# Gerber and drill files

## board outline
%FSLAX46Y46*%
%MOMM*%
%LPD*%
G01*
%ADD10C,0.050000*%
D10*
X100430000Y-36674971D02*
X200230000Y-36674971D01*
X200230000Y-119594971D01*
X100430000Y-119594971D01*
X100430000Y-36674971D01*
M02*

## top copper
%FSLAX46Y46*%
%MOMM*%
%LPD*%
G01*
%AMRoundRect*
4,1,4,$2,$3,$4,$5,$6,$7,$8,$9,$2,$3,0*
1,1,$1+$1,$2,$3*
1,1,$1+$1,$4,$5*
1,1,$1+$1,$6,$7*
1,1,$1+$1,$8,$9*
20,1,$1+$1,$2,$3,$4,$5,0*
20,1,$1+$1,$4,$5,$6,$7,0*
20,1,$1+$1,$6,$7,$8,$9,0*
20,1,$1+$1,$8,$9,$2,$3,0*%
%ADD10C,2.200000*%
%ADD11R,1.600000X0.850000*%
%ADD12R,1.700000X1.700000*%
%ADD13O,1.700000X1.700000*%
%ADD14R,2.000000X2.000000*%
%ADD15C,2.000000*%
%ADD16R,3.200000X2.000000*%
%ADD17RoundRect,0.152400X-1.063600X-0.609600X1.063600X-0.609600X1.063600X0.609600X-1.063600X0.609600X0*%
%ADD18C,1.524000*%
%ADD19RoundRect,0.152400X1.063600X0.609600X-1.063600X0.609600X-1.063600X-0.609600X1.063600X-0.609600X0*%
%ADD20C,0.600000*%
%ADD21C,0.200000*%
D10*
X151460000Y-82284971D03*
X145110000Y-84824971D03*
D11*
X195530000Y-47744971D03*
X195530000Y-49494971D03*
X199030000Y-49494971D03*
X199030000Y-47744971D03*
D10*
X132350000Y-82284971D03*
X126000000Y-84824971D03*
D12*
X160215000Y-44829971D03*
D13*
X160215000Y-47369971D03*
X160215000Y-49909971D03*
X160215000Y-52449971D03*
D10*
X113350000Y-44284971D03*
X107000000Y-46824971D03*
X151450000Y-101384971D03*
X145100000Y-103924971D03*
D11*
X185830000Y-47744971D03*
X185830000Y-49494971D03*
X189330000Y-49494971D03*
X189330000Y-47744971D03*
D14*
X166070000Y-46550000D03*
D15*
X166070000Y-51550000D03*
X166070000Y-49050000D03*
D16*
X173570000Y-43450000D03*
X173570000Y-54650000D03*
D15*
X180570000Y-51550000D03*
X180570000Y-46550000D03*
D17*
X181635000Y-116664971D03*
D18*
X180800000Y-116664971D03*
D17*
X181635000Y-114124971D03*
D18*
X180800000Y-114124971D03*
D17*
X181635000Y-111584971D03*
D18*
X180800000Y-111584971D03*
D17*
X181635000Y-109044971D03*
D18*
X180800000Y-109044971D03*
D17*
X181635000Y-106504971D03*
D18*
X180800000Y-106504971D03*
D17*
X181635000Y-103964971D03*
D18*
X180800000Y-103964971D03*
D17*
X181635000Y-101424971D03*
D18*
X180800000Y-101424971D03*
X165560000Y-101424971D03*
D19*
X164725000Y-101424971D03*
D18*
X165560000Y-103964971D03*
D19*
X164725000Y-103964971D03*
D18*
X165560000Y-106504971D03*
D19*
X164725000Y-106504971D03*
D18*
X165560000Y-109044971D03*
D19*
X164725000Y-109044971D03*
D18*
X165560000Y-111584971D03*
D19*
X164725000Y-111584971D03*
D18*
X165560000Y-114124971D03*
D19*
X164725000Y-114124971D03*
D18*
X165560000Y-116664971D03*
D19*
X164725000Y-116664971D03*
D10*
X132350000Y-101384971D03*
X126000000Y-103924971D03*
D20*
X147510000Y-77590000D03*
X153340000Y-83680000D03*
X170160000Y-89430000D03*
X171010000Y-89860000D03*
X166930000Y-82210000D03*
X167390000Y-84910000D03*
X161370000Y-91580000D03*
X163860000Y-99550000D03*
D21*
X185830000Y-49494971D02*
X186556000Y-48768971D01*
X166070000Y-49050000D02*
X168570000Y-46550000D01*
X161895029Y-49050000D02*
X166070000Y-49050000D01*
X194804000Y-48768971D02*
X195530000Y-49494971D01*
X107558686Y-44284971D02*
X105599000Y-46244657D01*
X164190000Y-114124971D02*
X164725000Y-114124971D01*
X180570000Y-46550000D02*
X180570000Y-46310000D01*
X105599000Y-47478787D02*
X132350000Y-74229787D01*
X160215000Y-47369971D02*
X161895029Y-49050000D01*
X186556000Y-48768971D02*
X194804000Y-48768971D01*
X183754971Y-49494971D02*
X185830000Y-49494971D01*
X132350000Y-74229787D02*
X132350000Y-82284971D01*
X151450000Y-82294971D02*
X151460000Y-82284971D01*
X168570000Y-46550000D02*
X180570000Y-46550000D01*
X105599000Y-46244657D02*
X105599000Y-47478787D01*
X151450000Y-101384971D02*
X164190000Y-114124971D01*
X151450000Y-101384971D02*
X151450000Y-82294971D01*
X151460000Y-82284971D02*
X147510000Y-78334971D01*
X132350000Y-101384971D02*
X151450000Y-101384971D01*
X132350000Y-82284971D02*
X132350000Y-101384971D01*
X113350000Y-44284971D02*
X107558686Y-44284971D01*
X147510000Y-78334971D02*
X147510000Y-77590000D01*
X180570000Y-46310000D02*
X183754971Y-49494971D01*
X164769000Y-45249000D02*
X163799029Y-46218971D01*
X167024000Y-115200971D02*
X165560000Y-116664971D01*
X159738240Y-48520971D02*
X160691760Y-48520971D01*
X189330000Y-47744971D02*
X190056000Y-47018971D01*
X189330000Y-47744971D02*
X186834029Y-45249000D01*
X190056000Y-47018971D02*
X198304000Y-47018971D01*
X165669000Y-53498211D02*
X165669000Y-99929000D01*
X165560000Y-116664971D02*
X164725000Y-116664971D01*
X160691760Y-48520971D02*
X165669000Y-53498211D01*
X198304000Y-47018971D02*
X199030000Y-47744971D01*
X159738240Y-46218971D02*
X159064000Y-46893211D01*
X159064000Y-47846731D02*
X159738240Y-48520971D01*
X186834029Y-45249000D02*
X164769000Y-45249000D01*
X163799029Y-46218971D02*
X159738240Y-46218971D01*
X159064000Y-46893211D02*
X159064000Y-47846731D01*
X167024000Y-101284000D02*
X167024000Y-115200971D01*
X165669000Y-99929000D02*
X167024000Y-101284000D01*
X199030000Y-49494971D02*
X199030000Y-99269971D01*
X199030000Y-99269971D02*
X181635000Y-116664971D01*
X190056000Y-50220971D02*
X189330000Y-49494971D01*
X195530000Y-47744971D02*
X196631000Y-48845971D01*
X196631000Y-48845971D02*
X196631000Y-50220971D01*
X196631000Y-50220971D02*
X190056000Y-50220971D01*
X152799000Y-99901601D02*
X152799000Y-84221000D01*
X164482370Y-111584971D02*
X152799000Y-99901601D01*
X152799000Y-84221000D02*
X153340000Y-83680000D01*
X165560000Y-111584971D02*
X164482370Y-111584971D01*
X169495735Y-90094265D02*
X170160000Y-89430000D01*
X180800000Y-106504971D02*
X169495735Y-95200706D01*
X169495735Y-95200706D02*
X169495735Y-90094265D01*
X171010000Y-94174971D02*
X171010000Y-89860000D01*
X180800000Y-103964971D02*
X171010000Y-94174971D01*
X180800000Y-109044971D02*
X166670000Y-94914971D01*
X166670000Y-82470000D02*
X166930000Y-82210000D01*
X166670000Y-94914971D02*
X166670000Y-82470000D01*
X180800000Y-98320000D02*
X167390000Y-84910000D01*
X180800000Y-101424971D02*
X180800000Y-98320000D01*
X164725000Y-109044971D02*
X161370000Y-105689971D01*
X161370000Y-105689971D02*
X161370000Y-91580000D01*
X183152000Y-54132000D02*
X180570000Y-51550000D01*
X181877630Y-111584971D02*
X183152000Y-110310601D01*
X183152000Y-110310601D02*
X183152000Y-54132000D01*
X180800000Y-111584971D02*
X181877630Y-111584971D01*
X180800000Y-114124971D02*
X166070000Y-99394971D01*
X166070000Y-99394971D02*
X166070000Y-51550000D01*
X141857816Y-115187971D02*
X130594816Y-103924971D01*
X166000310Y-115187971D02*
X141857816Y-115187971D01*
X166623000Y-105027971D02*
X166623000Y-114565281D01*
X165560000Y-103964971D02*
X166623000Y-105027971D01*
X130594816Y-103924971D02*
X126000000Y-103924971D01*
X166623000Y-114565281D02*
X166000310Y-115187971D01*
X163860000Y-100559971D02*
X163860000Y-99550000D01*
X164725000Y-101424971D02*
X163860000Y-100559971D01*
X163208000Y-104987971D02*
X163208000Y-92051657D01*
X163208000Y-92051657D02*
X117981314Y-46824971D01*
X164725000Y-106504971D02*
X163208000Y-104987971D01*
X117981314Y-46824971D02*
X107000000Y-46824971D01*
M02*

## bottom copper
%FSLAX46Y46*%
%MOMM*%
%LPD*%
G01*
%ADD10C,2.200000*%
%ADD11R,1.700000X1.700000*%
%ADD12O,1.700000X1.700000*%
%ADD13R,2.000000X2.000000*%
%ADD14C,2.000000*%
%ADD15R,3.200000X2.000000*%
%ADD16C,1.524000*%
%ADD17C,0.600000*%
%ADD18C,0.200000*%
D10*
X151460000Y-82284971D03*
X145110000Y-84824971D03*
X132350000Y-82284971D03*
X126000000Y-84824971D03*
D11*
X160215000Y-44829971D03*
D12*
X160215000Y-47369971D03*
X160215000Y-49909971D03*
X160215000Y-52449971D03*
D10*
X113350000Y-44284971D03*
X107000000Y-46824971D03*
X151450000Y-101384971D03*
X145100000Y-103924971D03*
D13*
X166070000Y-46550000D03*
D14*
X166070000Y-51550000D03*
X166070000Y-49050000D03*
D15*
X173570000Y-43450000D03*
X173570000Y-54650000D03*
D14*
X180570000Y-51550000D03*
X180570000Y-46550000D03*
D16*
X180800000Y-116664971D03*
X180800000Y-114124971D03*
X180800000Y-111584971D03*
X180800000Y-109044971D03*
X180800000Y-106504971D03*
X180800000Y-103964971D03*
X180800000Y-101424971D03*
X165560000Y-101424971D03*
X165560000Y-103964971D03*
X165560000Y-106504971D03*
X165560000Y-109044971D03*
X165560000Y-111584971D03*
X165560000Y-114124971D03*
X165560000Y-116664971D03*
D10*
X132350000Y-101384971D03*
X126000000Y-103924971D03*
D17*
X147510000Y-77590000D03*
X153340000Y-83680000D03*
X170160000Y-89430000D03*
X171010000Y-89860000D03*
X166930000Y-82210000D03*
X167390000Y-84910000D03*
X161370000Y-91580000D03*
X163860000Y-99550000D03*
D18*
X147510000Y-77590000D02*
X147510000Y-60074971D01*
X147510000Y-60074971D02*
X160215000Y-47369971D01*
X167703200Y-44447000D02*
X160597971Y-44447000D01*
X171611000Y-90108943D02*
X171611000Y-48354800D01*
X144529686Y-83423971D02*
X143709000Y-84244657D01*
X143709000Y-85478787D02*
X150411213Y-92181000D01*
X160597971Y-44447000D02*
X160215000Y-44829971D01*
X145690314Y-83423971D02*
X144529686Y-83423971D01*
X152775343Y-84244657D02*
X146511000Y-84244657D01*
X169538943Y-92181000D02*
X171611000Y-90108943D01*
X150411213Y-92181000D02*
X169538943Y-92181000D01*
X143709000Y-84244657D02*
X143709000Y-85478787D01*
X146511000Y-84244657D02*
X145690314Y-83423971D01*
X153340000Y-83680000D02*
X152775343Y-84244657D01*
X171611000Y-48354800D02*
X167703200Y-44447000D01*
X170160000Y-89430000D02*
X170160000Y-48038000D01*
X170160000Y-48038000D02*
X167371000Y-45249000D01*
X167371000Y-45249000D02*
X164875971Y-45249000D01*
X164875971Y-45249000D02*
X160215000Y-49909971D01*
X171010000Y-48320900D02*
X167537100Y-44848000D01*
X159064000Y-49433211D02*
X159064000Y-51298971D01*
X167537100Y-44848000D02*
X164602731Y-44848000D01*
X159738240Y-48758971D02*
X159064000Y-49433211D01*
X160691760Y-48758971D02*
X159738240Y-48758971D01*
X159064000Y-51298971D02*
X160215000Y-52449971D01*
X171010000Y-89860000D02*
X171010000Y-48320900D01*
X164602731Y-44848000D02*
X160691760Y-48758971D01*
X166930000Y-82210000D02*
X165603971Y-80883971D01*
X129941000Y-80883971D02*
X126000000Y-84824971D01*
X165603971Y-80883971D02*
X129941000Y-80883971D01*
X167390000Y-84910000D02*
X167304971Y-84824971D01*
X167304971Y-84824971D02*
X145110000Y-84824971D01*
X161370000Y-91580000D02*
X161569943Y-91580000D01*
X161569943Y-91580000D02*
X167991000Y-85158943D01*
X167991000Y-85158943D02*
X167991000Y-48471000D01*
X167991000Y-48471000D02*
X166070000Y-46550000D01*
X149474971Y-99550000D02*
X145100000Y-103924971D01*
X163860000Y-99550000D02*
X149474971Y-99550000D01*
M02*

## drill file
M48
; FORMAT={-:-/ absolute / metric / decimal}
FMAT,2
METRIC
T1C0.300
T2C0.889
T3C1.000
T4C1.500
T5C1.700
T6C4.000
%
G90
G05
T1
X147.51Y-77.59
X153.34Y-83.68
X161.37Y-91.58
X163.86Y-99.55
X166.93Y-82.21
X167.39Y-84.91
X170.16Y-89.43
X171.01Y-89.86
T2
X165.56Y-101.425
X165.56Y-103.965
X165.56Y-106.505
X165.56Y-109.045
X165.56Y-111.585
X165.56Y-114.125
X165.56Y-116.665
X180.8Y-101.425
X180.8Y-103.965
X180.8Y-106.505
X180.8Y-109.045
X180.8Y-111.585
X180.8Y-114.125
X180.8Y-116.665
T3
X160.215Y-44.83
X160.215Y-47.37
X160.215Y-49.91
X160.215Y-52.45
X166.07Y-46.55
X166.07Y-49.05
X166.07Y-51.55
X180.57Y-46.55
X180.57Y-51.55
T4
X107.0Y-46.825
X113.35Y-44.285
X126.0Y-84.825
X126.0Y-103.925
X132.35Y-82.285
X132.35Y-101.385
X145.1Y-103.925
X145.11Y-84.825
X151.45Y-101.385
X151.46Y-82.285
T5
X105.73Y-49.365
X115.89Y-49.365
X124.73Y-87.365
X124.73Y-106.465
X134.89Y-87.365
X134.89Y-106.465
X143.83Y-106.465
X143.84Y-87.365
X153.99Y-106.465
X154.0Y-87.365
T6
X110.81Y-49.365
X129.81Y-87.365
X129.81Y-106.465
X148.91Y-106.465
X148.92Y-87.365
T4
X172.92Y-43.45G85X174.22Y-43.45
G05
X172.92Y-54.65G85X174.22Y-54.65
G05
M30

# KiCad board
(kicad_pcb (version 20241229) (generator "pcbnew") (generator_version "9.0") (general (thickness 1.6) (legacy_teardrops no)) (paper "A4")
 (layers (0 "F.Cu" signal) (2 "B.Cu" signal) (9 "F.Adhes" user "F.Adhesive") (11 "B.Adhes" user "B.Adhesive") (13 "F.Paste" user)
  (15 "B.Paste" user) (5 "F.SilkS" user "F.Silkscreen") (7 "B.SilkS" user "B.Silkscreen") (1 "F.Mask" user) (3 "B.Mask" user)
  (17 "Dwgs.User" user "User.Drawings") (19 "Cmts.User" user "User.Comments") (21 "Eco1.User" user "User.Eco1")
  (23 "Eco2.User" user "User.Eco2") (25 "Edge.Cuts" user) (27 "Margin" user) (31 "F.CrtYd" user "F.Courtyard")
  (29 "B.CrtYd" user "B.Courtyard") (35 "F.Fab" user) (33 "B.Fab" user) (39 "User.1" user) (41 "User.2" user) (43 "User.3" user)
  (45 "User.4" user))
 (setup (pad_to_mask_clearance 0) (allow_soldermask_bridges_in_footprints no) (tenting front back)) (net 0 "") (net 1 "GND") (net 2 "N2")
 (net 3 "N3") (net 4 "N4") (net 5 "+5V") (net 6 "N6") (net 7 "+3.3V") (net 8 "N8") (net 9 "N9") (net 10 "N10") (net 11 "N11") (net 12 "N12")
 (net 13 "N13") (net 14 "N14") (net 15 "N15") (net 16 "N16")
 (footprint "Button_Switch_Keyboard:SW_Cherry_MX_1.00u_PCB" (layer "F.Cu") (at 151.46 82.284971)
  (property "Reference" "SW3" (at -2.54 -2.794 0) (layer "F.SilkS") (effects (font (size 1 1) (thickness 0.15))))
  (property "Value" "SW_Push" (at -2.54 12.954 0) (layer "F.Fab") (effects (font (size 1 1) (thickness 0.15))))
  (pad "" np_thru_hole circle (at -7.62 5.08) (size 1.7 1.7) (drill 1.7) (layers "*.Cu" "*.Mask"))
  (pad "" np_thru_hole circle (at -2.54 5.08) (size 4 4) (drill 4) (layers "*.Cu" "*.Mask"))
  (pad "" np_thru_hole circle (at 2.54 5.08) (size 1.7 1.7) (drill 1.7) (layers "*.Cu" "*.Mask"))
  (pad "1" thru_hole circle (at 0 0) (size 2.2 2.2) (drill 1.5) (layers "*.Cu" "*.Mask") (remove_unused_layers no) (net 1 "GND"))
  (pad "2" thru_hole circle (at -6.35 2.54) (size 2.2 2.2) (drill 1.5) (layers "*.Cu" "*.Mask") (remove_unused_layers no) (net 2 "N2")))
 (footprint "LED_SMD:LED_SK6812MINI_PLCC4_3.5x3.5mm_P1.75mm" (layer "F.Cu") (at 197.28 48.619971)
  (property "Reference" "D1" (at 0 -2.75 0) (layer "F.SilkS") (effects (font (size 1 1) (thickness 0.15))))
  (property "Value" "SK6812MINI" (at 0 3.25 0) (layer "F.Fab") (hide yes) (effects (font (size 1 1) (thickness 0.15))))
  (pad "1" smd rect (at -1.75 -0.875) (size 1.6 0.85) (layers "F.Cu" "F.Mask" "F.Paste") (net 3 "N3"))
  (pad "2" smd rect (at -1.75 0.875) (size 1.6 0.85) (layers "F.Cu" "F.Mask" "F.Paste") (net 1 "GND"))
  (pad "3" smd rect (at 1.75 0.875) (size 1.6 0.85) (layers "F.Cu" "F.Mask" "F.Paste") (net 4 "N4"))
  (pad "4" smd rect (at 1.75 -0.875) (size 1.6 0.85) (layers "F.Cu" "F.Mask" "F.Paste") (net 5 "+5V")))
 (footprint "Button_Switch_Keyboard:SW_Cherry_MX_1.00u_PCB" (layer "F.Cu") (at 132.35 82.284971)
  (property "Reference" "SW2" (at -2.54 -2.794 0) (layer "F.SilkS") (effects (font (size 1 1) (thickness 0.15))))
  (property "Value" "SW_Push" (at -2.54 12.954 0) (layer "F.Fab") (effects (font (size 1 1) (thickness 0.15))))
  (pad "" np_thru_hole circle (at -7.62 5.08) (size 1.7 1.7) (drill 1.7) (layers "*.Cu" "*.Mask"))
  (pad "" np_thru_hole circle (at -2.54 5.08) (size 4 4) (drill 4) (layers "*.Cu" "*.Mask"))
  (pad "" np_thru_hole circle (at 2.54 5.08) (size 1.7 1.7) (drill 1.7) (layers "*.Cu" "*.Mask"))
  (pad "1" thru_hole circle (at 0 0) (size 2.2 2.2) (drill 1.5) (layers "*.Cu" "*.Mask") (remove_unused_layers no) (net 1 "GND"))
  (pad "2" thru_hole circle (at -6.35 2.54) (size 2.2 2.2) (drill 1.5) (layers "*.Cu" "*.Mask") (remove_unused_layers no) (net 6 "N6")))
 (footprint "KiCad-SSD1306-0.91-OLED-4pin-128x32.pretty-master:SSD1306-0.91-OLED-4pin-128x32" (layer "F.Cu") (at 123.715 42.639971)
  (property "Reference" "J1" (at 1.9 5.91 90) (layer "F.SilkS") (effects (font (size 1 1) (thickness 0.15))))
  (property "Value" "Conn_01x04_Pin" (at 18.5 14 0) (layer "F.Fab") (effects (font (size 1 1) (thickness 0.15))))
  (pad "1" thru_hole rect (at 36.5 2.19) (size 1.7 1.7) (drill 1) (layers "*.Cu" "*.Mask") (remove_unused_layers no) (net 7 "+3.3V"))
  (pad "2" thru_hole oval (at 36.5 4.73) (size 1.7 1.7) (drill 1) (layers "*.Cu" "*.Mask") (remove_unused_layers no) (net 1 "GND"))
  (pad "3" thru_hole oval (at 36.5 7.27) (size 1.7 1.7) (drill 1) (layers "*.Cu" "*.Mask") (remove_unused_layers no) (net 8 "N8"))
  (pad "4" thru_hole oval (at 36.5 9.81) (size 1.7 1.7) (drill 1) (layers "*.Cu" "*.Mask") (remove_unused_layers no) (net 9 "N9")))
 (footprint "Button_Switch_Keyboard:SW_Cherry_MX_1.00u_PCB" (layer "F.Cu") (at 113.35 44.284971)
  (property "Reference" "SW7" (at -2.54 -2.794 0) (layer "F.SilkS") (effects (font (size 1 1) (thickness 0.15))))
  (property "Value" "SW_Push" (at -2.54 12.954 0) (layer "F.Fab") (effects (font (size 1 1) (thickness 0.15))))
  (pad "" np_thru_hole circle (at -7.62 5.08) (size 1.7 1.7) (drill 1.7) (layers "*.Cu" "*.Mask"))
  (pad "" np_thru_hole circle (at -2.54 5.08) (size 4 4) (drill 4) (layers "*.Cu" "*.Mask"))
  (pad "" np_thru_hole circle (at 2.54 5.08) (size 1.7 1.7) (drill 1.7) (layers "*.Cu" "*.Mask"))
  (pad "1" thru_hole circle (at 0 0) (size 2.2 2.2) (drill 1.5) (layers "*.Cu" "*.Mask") (remove_unused_layers no) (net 1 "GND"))
  (pad "2" thru_hole circle (at -6.35 2.54) (size 2.2 2.2) (drill 1.5) (layers "*.Cu" "*.Mask") (remove_unused_layers no) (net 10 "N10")))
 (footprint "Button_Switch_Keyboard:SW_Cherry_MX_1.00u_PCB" (layer "F.Cu") (at 151.45 101.384971)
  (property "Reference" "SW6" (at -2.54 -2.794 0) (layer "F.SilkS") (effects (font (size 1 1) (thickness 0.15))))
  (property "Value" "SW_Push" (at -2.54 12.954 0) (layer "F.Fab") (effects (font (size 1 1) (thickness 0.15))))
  (pad "" np_thru_hole circle (at -7.62 5.08) (size 1.7 1.7) (drill 1.7) (layers "*.Cu" "*.Mask"))
  (pad "" np_thru_hole circle (at -2.54 5.08) (size 4 4) (drill 4) (layers "*.Cu" "*.Mask"))
  (pad "" np_thru_hole circle (at 2.54 5.08) (size 1.7 1.7) (drill 1.7) (layers "*.Cu" "*.Mask"))
  (pad "1" thru_hole circle (at 0 0) (size 2.2 2.2) (drill 1.5) (layers "*.Cu" "*.Mask") (remove_unused_layers no) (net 1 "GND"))
  (pad "2" thru_hole circle (at -6.35 2.54) (size 2.2 2.2) (drill 1.5) (layers "*.Cu" "*.Mask") (remove_unused_layers no) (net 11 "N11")))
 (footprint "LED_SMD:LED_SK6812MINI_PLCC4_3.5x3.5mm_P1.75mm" (layer "F.Cu") (at 187.58 48.619971)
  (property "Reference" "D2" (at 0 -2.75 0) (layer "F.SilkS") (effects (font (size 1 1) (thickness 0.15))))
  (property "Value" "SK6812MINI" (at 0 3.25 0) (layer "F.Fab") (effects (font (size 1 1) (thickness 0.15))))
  (pad "1" smd rect (at -1.75 -0.875) (size 1.6 0.85) (layers "F.Cu" "F.Mask" "F.Paste") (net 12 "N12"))
  (pad "2" smd rect (at -1.75 0.875) (size 1.6 0.85) (layers "F.Cu" "F.Mask" "F.Paste") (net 1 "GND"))
  (pad "3" smd rect (at 1.75 0.875) (size 1.6 0.85) (layers "F.Cu" "F.Mask" "F.Paste") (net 3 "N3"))
  (pad "4" smd rect (at 1.75 -0.875) (size 1.6 0.85) (layers "F.Cu" "F.Mask" "F.Paste") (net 5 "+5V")))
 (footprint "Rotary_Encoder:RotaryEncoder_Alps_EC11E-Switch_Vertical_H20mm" (layer "F.Cu") (at 166.07 46.55)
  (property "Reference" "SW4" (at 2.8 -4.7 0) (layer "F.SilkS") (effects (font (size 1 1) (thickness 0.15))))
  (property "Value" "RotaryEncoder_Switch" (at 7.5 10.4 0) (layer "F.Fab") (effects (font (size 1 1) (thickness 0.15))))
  (pad "A" thru_hole rect (at 0 0) (size 2 2) (drill 1) (layers "*.Cu" "*.Mask") (remove_unused_layers no) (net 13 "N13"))
  (pad "B" thru_hole circle (at 0 5) (size 2 2) (drill 1) (layers "*.Cu" "*.Mask") (remove_unused_layers no) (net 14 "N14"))
  (pad "C" thru_hole circle (at 0 2.5) (size 2 2) (drill 1) (layers "*.Cu" "*.Mask") (remove_unused_layers no) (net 1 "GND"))
  (pad "MP" thru_hole rect (at 7.5 -3.1) (size 3.2 2) (drill oval 2.8 1.5) (layers "*.Cu" "*.Mask") (remove_unused_layers no))
  (pad "MP" thru_hole rect (at 7.5 8.1) (size 3.2 2) (drill oval 2.8 1.5) (layers "*.Cu" "*.Mask") (remove_unused_layers no))
  (pad "S1" thru_hole circle (at 14.5 5) (size 2 2) (drill 1) (layers "*.Cu" "*.Mask") (remove_unused_layers no) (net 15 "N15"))
  (pad "S2" thru_hole circle (at 14.5 0) (size 2 2) (drill 1) (layers "*.Cu" "*.Mask") (remove_unused_layers no) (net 1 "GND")))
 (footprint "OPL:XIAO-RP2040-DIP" (layer "F.Cu") (at 173.18 109.044971 180)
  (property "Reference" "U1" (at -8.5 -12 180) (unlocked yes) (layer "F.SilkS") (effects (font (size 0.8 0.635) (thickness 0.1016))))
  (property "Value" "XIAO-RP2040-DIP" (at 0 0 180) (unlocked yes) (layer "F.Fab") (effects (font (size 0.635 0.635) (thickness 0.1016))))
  (pad "1" smd roundrect (at -8.455 -7.62) (size 2.432 1.524) (layers "F.Cu" "F.Mask") (roundrect_rratio 0.1) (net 4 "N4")
   (thermal_bridge_angle 45))
  (pad "1" thru_hole circle (at -7.62 -7.62) (size 1.524 1.524) (drill 0.889) (layers "*.Cu" "*.Mask") (remove_unused_layers no)
   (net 4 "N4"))
  (pad "2" smd roundrect (at -8.455 -5.08) (size 2.432 1.524) (layers "F.Cu" "F.Mask") (roundrect_rratio 0.1) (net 14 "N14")
   (thermal_bridge_angle 45))
  (pad "2" thru_hole circle (at -7.62 -5.08) (size 1.524 1.524) (drill 0.889) (layers "*.Cu" "*.Mask") (remove_unused_layers no)
   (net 14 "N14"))
  (pad "3" smd roundrect (at -8.455 -2.54) (size 2.432 1.524) (layers "F.Cu" "F.Mask") (roundrect_rratio 0.1) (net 15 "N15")
   (thermal_bridge_angle 45))
  (pad "3" thru_hole circle (at -7.62 -2.54) (size 1.524 1.524) (drill 0.889) (layers "*.Cu" "*.Mask") (remove_unused_layers no)
   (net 15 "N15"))
  (pad "4" smd roundrect (at -8.455 0) (size 2.432 1.524) (layers "F.Cu" "F.Mask") (roundrect_rratio 0.1) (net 6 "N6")
   (thermal_bridge_angle 45))
  (pad "4" thru_hole circle (at -7.62 0) (size 1.524 1.524) (drill 0.889) (layers "*.Cu" "*.Mask") (remove_unused_layers no) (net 6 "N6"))
  (pad "5" smd roundrect (at -8.455 2.54) (size 2.432 1.524) (layers "F.Cu" "F.Mask") (roundrect_rratio 0.1) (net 8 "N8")
   (thermal_bridge_angle 45))
  (pad "5" thru_hole circle (at -7.62 2.54) (size 1.524 1.524) (drill 0.889) (layers "*.Cu" "*.Mask") (remove_unused_layers no) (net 8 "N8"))
  (pad "6" smd roundrect (at -8.455 5.08) (size 2.432 1.524) (layers "F.Cu" "F.Mask") (roundrect_rratio 0.1) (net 9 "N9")
   (thermal_bridge_angle 45))
  (pad "6" thru_hole circle (at -7.62 5.08) (size 1.524 1.524) (drill 0.889) (layers "*.Cu" "*.Mask") (remove_unused_layers no) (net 9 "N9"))
  (pad "7" smd roundrect (at -8.455 7.62) (size 2.432 1.524) (layers "F.Cu" "F.Mask") (roundrect_rratio 0.1) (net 2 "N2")
   (thermal_bridge_angle 45))
  (pad "7" thru_hole circle (at -7.62 7.62) (size 1.524 1.524) (drill 0.889) (layers "*.Cu" "*.Mask") (remove_unused_layers no) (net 2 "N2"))
  (pad "8" thru_hole circle (at 7.62 7.62 180) (size 1.524 1.524) (drill 0.889) (layers "*.Cu" "*.Mask") (remove_unused_layers no)
   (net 11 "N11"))
  (pad "8" smd roundrect (at 8.455 7.62 180) (size 2.432 1.524) (layers "F.Cu" "F.Mask") (roundrect_rratio 0.1) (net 11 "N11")
   (thermal_bridge_angle 45))
  (pad "9" thru_hole circle (at 7.62 5.08 180) (size 1.524 1.524) (drill 0.889) (layers "*.Cu" "*.Mask") (remove_unused_layers no)
   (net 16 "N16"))
  (pad "9" smd roundrect (at 8.455 5.08 180) (size 2.432 1.524) (layers "F.Cu" "F.Mask") (roundrect_rratio 0.1) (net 16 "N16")
   (thermal_bridge_angle 45))
  (pad "10" thru_hole circle (at 7.62 2.54 180) (size 1.524 1.524) (drill 0.889) (layers "*.Cu" "*.Mask") (remove_unused_layers no)
   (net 10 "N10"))
  (pad "10" smd roundrect (at 8.455 2.54 180) (size 2.432 1.524) (layers "F.Cu" "F.Mask") (roundrect_rratio 0.1) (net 10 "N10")
   (thermal_bridge_angle 45))
  (pad "11" thru_hole circle (at 7.62 0 180) (size 1.524 1.524) (drill 0.889) (layers "*.Cu" "*.Mask") (remove_unused_layers no)
   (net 13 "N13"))
  (pad "11" smd roundrect (at 8.455 0 180) (size 2.432 1.524) (layers "F.Cu" "F.Mask") (roundrect_rratio 0.1) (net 13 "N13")
   (thermal_bridge_angle 45))
  (pad "12" thru_hole circle (at 7.62 -2.54 180) (size 1.524 1.524) (drill 0.889) (layers "*.Cu" "*.Mask") (remove_unused_layers no)
   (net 7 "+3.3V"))
  (pad "12" smd roundrect (at 8.455 -2.54 180) (size 2.432 1.524) (layers "F.Cu" "F.Mask") (roundrect_rratio 0.1) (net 7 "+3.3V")
   (thermal_bridge_angle 45))
  (pad "13" thru_hole circle (at 7.62 -5.08 180) (size 1.524 1.524) (drill 0.889) (layers "*.Cu" "*.Mask") (remove_unused_layers no)
   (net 1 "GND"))
  (pad "13" smd roundrect (at 8.455 -5.08 180) (size 2.432 1.524) (layers "F.Cu" "F.Mask") (roundrect_rratio 0.1) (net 1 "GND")
   (thermal_bridge_angle 45))
  (pad "14" thru_hole circle (at 7.62 -7.62 180) (size 1.524 1.524) (drill 0.889) (layers "*.Cu" "*.Mask") (remove_unused_layers no)
   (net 5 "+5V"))
  (pad "14" smd roundrect (at 8.455 -7.62 180) (size 2.432 1.524) (layers "F.Cu" "F.Mask") (roundrect_rratio 0.1) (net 5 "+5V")
   (thermal_bridge_angle 45)))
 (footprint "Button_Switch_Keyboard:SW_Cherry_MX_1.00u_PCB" (layer "F.Cu") (at 132.35 101.384971)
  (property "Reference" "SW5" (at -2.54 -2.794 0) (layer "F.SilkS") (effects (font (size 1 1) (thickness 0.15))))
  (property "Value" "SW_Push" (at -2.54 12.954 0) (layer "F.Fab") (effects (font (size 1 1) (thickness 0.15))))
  (pad "" np_thru_hole circle (at -7.62 5.08) (size 1.7 1.7) (drill 1.7) (layers "*.Cu" "*.Mask"))
  (pad "" np_thru_hole circle (at -2.54 5.08) (size 4 4) (drill 4) (layers "*.Cu" "*.Mask"))
  (pad "" np_thru_hole circle (at 2.54 5.08) (size 1.7 1.7) (drill 1.7) (layers "*.Cu" "*.Mask"))
  (pad "1" thru_hole circle (at 0 0) (size 2.2 2.2) (drill 1.5) (layers "*.Cu" "*.Mask") (remove_unused_layers no) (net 1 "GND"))
  (pad "2" thru_hole circle (at -6.35 2.54) (size 2.2 2.2) (drill 1.5) (layers "*.Cu" "*.Mask") (remove_unused_layers no) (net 16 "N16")))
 (gr_rect (start 100.43 36.674971) (end 200.23 119.594971) (stroke (width 0.05) (type default)) (fill no) (layer "Edge.Cuts"))
 (segment (start 185.83 49.494971) (end 186.556 48.768971) (width 0.2) (layer "F.Cu") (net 1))
 (segment (start 166.07 49.05) (end 168.57 46.55) (width 0.2) (layer "F.Cu") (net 1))
 (segment (start 161.895029 49.05) (end 166.07 49.05) (width 0.2) (layer "F.Cu") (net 1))
 (segment (start 194.804 48.768971) (end 195.53 49.494971) (width 0.2) (layer "F.Cu") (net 1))
 (segment (start 107.558686 44.284971) (end 105.599 46.244657) (width 0.2) (layer "F.Cu") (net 1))
 (segment (start 164.19 114.124971) (end 164.725 114.124971) (width 0.2) (layer "F.Cu") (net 1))
 (segment (start 180.57 46.55) (end 180.57 46.31) (width 0.2) (layer "F.Cu") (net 1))
 (segment (start 105.599 47.478787) (end 132.35 74.229787) (width 0.2) (layer "F.Cu") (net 1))
 (segment (start 160.215 47.369971) (end 161.895029 49.05) (width 0.2) (layer "F.Cu") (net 1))
 (segment (start 186.556 48.768971) (end 194.804 48.768971) (width 0.2) (layer "F.Cu") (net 1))
 (segment (start 183.754971 49.494971) (end 185.83 49.494971) (width 0.2) (layer "F.Cu") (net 1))
 (segment (start 132.35 74.229787) (end 132.35 82.284971) (width 0.2) (layer "F.Cu") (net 1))
 (segment (start 151.45 82.294971) (end 151.46 82.284971) (width 0.2) (layer "F.Cu") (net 1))
 (segment (start 168.57 46.55) (end 180.57 46.55) (width 0.2) (layer "F.Cu") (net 1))
 (segment (start 105.599 46.244657) (end 105.599 47.478787) (width 0.2) (layer "F.Cu") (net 1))
 (segment (start 151.45 101.384971) (end 164.19 114.124971) (width 0.2) (layer "F.Cu") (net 1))
 (segment (start 151.45 101.384971) (end 151.45 82.294971) (width 0.2) (layer "F.Cu") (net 1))
 (segment (start 151.46 82.284971) (end 147.51 78.334971) (width 0.2) (layer "F.Cu") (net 1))
 (segment (start 132.35 101.384971) (end 151.45 101.384971) (width 0.2) (layer "F.Cu") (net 1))
 (segment (start 132.35 82.284971) (end 132.35 101.384971) (width 0.2) (layer "F.Cu") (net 1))
 (segment (start 113.35 44.284971) (end 107.558686 44.284971) (width 0.2) (layer "F.Cu") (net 1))
 (segment (start 147.51 78.334971) (end 147.51 77.59) (width 0.2) (layer "F.Cu") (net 1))
 (segment (start 180.57 46.31) (end 183.754971 49.494971) (width 0.2) (layer "F.Cu") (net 1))
 (via (at 147.51 77.59) (size 0.6) (drill 0.3) (layers "F.Cu" "B.Cu") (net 1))
 (segment (start 147.51 77.59) (end 147.51 60.074971) (width 0.2) (layer "B.Cu") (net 1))
 (segment (start 147.51 60.074971) (end 160.215 47.369971) (width 0.2) (layer "B.Cu") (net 1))
 (segment (start 164.769 45.249) (end 163.799029 46.218971) (width 0.2) (layer "F.Cu") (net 5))
 (segment (start 167.024 115.200971) (end 165.56 116.664971) (width 0.2) (layer "F.Cu") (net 5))
 (segment (start 159.73824 48.520971) (end 160.69176 48.520971) (width 0.2) (layer "F.Cu") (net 5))
 (segment (start 189.33 47.744971) (end 190.056 47.018971) (width 0.2) (layer "F.Cu") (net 5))
 (segment (start 189.33 47.744971) (end 186.834029 45.249) (width 0.2) (layer "F.Cu") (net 5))
 (segment (start 190.056 47.018971) (end 198.304 47.018971) (width 0.2) (layer "F.Cu") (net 5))
 (segment (start 165.669 53.498211) (end 165.669 99.929) (width 0.2) (layer "F.Cu") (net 5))
 (segment (start 165.56 116.664971) (end 164.725 116.664971) (width 0.2) (layer "F.Cu") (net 5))
 (segment (start 160.69176 48.520971) (end 165.669 53.498211) (width 0.2) (layer "F.Cu") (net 5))
 (segment (start 198.304 47.018971) (end 199.03 47.744971) (width 0.2) (layer "F.Cu") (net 5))
 (segment (start 159.73824 46.218971) (end 159.064 46.893211) (width 0.2) (layer "F.Cu") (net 5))
 (segment (start 159.064 47.846731) (end 159.73824 48.520971) (width 0.2) (layer "F.Cu") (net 5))
 (segment (start 186.834029 45.249) (end 164.769 45.249) (width 0.2) (layer "F.Cu") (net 5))
 (segment (start 163.799029 46.218971) (end 159.73824 46.218971) (width 0.2) (layer "F.Cu") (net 5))
 (segment (start 159.064 46.893211) (end 159.064 47.846731) (width 0.2) (layer "F.Cu") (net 5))
 (segment (start 167.024 101.284) (end 167.024 115.200971) (width 0.2) (layer "F.Cu") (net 5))
 (segment (start 165.669 99.929) (end 167.024 101.284) (width 0.2) (layer "F.Cu") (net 5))
 (segment (start 199.03 49.494971) (end 199.03 99.269971) (width 0.2) (layer "F.Cu") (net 4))
 (segment (start 199.03 99.269971) (end 181.635 116.664971) (width 0.2) (layer "F.Cu") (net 4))
 (segment (start 190.056 50.220971) (end 189.33 49.494971) (width 0.2) (layer "F.Cu") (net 3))
 (segment (start 195.53 47.744971) (end 196.631 48.845971) (width 0.2) (layer "F.Cu") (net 3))
 (segment (start 196.631 48.845971) (end 196.631 50.220971) (width 0.2) (layer "F.Cu") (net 3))
 (segment (start 196.631 50.220971) (end 190.056 50.220971) (width 0.2) (layer "F.Cu") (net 3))
 (segment (start 152.799 99.901601) (end 152.799 84.221) (width 0.2) (layer "F.Cu") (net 7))
 (segment (start 164.48237 111.584971) (end 152.799 99.901601) (width 0.2) (layer "F.Cu") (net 7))
 (segment (start 152.799 84.221) (end 153.34 83.68) (width 0.2) (layer "F.Cu") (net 7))
 (segment (start 165.56 111.584971) (end 164.48237 111.584971) (width 0.2) (layer "F.Cu") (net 7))
 (via (at 153.34 83.68) (size 0.6) (drill 0.3) (layers "F.Cu" "B.Cu") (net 7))
 (segment (start 167.7032 44.447) (end 160.597971 44.447) (width 0.2) (layer "B.Cu") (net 7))
 (segment (start 171.611 90.108943) (end 171.611 48.3548) (width 0.2) (layer "B.Cu") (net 7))
 (segment (start 144.529686 83.423971) (end 143.709 84.244657) (width 0.2) (layer "B.Cu") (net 7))
 (segment (start 143.709 85.478787) (end 150.411213 92.181) (width 0.2) (layer "B.Cu") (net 7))
 (segment (start 160.597971 44.447) (end 160.215 44.829971) (width 0.2) (layer "B.Cu") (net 7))
 (segment (start 145.690314 83.423971) (end 144.529686 83.423971) (width 0.2) (layer "B.Cu") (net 7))
 (segment (start 152.775343 84.244657) (end 146.511 84.244657) (width 0.2) (layer "B.Cu") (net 7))
 (segment (start 169.538943 92.181) (end 171.611 90.108943) (width 0.2) (layer "B.Cu") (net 7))
 (segment (start 150.411213 92.181) (end 169.538943 92.181) (width 0.2) (layer "B.Cu") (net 7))
 (segment (start 143.709 84.244657) (end 143.709 85.478787) (width 0.2) (layer "B.Cu") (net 7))
 (segment (start 146.511 84.244657) (end 145.690314 83.423971) (width 0.2) (layer "B.Cu") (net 7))
 (segment (start 153.34 83.68) (end 152.775343 84.244657) (width 0.2) (layer "B.Cu") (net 7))
 (segment (start 171.611 48.3548) (end 167.7032 44.447) (width 0.2) (layer "B.Cu") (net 7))
 (segment (start 169.495735 90.094265) (end 170.16 89.43) (width 0.2) (layer "F.Cu") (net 8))
 (segment (start 180.8 106.504971) (end 169.495735 95.200706) (width 0.2) (layer "F.Cu") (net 8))
 (segment (start 169.495735 95.200706) (end 169.495735 90.094265) (width 0.2) (layer "F.Cu") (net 8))
 (via (at 170.16 89.43) (size 0.6) (drill 0.3) (layers "F.Cu" "B.Cu") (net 8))
 (segment (start 170.16 89.43) (end 170.16 48.038) (width 0.2) (layer "B.Cu") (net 8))
 (segment (start 170.16 48.038) (end 167.371 45.249) (width 0.2) (layer "B.Cu") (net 8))
 (segment (start 167.371 45.249) (end 164.875971 45.249) (width 0.2) (layer "B.Cu") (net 8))
 (segment (start 164.875971 45.249) (end 160.215 49.909971) (width 0.2) (layer "B.Cu") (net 8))
 (segment (start 171.01 94.174971) (end 171.01 89.86) (width 0.2) (layer "F.Cu") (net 9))
 (segment (start 180.8 103.964971) (end 171.01 94.174971) (width 0.2) (layer "F.Cu") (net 9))
 (via (at 171.01 89.86) (size 0.6) (drill 0.3) (layers "F.Cu" "B.Cu") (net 9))
 (segment (start 171.01 48.3209) (end 167.5371 44.848) (width 0.2) (layer "B.Cu") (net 9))
 (segment (start 159.064 49.433211) (end 159.064 51.298971) (width 0.2) (layer "B.Cu") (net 9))
 (segment (start 167.5371 44.848) (end 164.602731 44.848) (width 0.2) (layer "B.Cu") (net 9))
 (segment (start 159.73824 48.758971) (end 159.064 49.433211) (width 0.2) (layer "B.Cu") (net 9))
 (segment (start 160.69176 48.758971) (end 159.73824 48.758971) (width 0.2) (layer "B.Cu") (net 9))
 (segment (start 159.064 51.298971) (end 160.215 52.449971) (width 0.2) (layer "B.Cu") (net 9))
 (segment (start 171.01 89.86) (end 171.01 48.3209) (width 0.2) (layer "B.Cu") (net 9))
 (segment (start 164.602731 44.848) (end 160.69176 48.758971) (width 0.2) (layer "B.Cu") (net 9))
 (segment (start 180.8 109.044971) (end 166.67 94.914971) (width 0.2) (layer "F.Cu") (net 6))
 (segment (start 166.67 82.47) (end 166.93 82.21) (width 0.2) (layer "F.Cu") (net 6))
 (segment (start 166.67 94.914971) (end 166.67 82.47) (width 0.2) (layer "F.Cu") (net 6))
 (via (at 166.93 82.21) (size 0.6) (drill 0.3) (layers "F.Cu" "B.Cu") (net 6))
 (segment (start 166.93 82.21) (end 165.603971 80.883971) (width 0.2) (layer "B.Cu") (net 6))
 (segment (start 129.941 80.883971) (end 126 84.824971) (width 0.2) (layer "B.Cu") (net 6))
 (segment (start 165.603971 80.883971) (end 129.941 80.883971) (width 0.2) (layer "B.Cu") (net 6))
 (segment (start 180.8 98.32) (end 167.39 84.91) (width 0.2) (layer "F.Cu") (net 2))
 (segment (start 180.8 101.424971) (end 180.8 98.32) (width 0.2) (layer "F.Cu") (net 2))
 (via (at 167.39 84.91) (size 0.6) (drill 0.3) (layers "F.Cu" "B.Cu") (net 2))
 (segment (start 167.39 84.91) (end 167.304971 84.824971) (width 0.2) (layer "B.Cu") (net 2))
 (segment (start 167.304971 84.824971) (end 145.11 84.824971) (width 0.2) (layer "B.Cu") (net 2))
 (segment (start 164.725 109.044971) (end 161.37 105.689971) (width 0.2) (layer "F.Cu") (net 13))
 (segment (start 161.37 105.689971) (end 161.37 91.58) (width 0.2) (layer "F.Cu") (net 13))
 (via (at 161.37 91.58) (size 0.6) (drill 0.3) (layers "F.Cu" "B.Cu") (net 13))
 (segment (start 161.37 91.58) (end 161.569943 91.58) (width 0.2) (layer "B.Cu") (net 13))
 (segment (start 161.569943 91.58) (end 167.991 85.158943) (width 0.2) (layer "B.Cu") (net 13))
 (segment (start 167.991 85.158943) (end 167.991 48.471) (width 0.2) (layer "B.Cu") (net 13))
 (segment (start 167.991 48.471) (end 166.07 46.55) (width 0.2) (layer "B.Cu") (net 13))
 (segment (start 183.152 54.132) (end 180.57 51.55) (width 0.2) (layer "F.Cu") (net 15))
 (segment (start 181.87763 111.584971) (end 183.152 110.310601) (width 0.2) (layer "F.Cu") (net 15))
 (segment (start 183.152 110.310601) (end 183.152 54.132) (width 0.2) (layer "F.Cu") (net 15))
 (segment (start 180.8 111.584971) (end 181.87763 111.584971) (width 0.2) (layer "F.Cu") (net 15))
 (segment (start 180.8 114.124971) (end 166.07 99.394971) (width 0.2) (layer "F.Cu") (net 14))
 (segment (start 166.07 99.394971) (end 166.07 51.55) (width 0.2) (layer "F.Cu") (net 14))
 (segment (start 141.857816 115.187971) (end 130.594816 103.924971) (width 0.2) (layer "F.Cu") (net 16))
 (segment (start 166.00031 115.187971) (end 141.857816 115.187971) (width 0.2) (layer "F.Cu") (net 16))
 (segment (start 166.623 105.027971) (end 166.623 114.565281) (width 0.2) (layer "F.Cu") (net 16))
 (segment (start 165.56 103.964971) (end 166.623 105.027971) (width 0.2) (layer "F.Cu") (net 16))
 (segment (start 130.594816 103.924971) (end 126 103.924971) (width 0.2) (layer "F.Cu") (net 16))
 (segment (start 166.623 114.565281) (end 166.00031 115.187971) (width 0.2) (layer "F.Cu") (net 16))
 (segment (start 163.86 100.559971) (end 163.86 99.55) (width 0.2) (layer "F.Cu") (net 11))
 (segment (start 164.725 101.424971) (end 163.86 100.559971) (width 0.2) (layer "F.Cu") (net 11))
 (via (at 163.86 99.55) (size 0.6) (drill 0.3) (layers "F.Cu" "B.Cu") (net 11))
 (segment (start 149.474971 99.55) (end 145.1 103.924971) (width 0.2) (layer "B.Cu") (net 11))
 (segment (start 163.86 99.55) (end 149.474971 99.55) (width 0.2) (layer "B.Cu") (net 11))
 (segment (start 163.208 104.987971) (end 163.208 92.051657) (width 0.2) (layer "F.Cu") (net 10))
 (segment (start 163.208 92.051657) (end 117.981314 46.824971) (width 0.2) (layer "F.Cu") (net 10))
 (segment (start 164.725 106.504971) (end 163.208 104.987971) (width 0.2) (layer "F.Cu") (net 10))
 (segment (start 117.981314 46.824971) (end 107 46.824971) (width 0.2) (layer "F.Cu") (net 10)))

